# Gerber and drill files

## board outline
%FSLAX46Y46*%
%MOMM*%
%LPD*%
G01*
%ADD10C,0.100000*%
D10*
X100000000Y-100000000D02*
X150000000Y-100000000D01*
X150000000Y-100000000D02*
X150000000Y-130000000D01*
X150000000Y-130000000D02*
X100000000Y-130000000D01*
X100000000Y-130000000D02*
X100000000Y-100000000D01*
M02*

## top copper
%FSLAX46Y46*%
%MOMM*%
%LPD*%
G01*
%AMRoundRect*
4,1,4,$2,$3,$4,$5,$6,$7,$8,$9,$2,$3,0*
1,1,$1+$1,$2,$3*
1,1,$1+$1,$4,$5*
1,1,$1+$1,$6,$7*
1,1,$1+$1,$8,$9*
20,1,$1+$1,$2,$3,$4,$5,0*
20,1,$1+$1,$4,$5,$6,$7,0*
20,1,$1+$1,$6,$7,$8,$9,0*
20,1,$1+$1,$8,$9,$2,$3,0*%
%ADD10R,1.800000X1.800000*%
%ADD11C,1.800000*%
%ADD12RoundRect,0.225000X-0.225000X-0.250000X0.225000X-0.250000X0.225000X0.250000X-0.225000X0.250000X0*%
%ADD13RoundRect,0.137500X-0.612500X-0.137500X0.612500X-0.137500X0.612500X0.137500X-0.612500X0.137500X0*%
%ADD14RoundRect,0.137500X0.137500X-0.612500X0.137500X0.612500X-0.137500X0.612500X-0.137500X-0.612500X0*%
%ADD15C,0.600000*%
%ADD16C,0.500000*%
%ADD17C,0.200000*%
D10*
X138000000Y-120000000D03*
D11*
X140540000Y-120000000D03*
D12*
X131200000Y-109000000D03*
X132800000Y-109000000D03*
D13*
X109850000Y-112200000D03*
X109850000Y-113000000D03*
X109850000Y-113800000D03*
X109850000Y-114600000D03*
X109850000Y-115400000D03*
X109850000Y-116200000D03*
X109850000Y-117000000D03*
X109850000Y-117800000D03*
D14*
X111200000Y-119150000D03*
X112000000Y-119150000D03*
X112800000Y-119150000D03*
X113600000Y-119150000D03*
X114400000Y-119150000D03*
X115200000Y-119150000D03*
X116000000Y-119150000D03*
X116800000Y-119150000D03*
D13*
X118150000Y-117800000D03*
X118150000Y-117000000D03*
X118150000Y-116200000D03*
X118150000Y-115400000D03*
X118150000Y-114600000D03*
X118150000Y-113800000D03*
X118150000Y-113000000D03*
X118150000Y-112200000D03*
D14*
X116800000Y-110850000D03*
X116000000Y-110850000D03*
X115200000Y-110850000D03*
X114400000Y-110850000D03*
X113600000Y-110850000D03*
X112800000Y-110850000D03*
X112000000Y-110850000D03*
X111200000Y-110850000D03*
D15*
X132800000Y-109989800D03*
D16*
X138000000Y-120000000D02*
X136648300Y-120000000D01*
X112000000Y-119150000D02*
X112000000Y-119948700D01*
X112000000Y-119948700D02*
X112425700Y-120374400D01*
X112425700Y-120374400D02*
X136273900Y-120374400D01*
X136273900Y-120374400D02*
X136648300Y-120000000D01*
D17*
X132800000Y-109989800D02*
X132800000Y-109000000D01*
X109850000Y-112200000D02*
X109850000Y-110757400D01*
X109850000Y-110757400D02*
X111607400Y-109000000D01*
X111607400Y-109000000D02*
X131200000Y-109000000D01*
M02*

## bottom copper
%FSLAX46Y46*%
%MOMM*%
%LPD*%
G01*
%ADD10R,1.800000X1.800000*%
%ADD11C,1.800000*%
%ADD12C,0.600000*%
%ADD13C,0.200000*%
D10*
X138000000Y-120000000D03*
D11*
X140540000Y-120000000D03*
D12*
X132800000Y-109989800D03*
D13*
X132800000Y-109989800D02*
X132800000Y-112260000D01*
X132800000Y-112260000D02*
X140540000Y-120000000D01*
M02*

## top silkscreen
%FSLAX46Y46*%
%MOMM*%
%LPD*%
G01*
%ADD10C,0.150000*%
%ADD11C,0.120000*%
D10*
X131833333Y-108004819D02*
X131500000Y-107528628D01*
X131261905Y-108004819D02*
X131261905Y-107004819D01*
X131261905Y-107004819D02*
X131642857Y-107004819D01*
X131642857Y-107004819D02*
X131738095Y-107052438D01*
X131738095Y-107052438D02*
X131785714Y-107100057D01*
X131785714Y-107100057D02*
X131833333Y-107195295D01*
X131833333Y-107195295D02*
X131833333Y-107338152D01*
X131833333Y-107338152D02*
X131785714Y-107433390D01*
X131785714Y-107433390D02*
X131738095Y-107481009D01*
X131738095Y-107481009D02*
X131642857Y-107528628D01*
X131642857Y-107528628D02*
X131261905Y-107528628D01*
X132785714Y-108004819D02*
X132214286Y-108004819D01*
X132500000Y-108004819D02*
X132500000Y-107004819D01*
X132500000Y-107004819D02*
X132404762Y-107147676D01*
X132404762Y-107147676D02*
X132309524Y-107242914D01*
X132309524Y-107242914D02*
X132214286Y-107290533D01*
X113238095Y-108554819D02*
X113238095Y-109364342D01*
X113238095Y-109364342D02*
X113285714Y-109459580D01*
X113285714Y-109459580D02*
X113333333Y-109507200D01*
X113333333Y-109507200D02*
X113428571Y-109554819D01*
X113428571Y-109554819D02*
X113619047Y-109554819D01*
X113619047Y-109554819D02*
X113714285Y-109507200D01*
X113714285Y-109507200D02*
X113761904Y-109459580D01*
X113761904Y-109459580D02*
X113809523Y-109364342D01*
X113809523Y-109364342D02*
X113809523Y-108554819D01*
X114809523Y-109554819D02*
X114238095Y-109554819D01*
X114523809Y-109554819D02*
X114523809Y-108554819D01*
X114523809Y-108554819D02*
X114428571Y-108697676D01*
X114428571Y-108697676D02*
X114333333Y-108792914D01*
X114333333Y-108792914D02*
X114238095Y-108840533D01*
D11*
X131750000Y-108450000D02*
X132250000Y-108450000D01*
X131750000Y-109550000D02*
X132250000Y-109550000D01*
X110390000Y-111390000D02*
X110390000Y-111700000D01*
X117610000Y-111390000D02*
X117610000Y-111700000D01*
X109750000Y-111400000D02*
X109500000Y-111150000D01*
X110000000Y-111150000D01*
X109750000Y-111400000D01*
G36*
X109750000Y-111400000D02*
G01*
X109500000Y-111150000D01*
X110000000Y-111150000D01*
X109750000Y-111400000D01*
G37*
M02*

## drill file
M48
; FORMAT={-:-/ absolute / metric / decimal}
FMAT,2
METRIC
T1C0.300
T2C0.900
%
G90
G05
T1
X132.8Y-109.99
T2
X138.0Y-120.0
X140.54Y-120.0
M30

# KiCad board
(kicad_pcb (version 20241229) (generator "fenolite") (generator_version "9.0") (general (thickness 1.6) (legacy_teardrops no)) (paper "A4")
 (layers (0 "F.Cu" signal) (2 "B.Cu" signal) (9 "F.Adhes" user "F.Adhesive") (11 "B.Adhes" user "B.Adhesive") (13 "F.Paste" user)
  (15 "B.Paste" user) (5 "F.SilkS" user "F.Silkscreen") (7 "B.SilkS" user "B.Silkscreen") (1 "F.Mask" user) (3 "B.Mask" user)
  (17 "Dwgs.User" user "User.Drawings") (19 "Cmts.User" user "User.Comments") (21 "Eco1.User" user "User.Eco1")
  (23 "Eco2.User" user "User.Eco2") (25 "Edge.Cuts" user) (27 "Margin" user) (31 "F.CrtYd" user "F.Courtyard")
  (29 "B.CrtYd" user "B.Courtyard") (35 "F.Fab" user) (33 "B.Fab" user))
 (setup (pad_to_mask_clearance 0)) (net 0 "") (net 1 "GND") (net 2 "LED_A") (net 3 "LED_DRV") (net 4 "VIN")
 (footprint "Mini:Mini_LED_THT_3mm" (layer "B.Cu") (at 138 120)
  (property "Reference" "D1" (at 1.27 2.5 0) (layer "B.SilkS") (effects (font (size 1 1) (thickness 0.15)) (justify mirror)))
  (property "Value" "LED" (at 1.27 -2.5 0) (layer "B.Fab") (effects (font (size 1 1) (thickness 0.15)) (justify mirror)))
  (pad "1" thru_hole rect (at 0 0) (size 1.8 1.8) (drill 0.9) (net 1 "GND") (layers "*.Cu" "*.Mask") (remove_unused_layers no))
  (pad "2" thru_hole circle (at 2.54 0) (size 1.8 1.8) (drill 0.9) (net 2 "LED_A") (layers "*.Cu" "*.Mask") (remove_unused_layers no)))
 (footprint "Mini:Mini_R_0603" (layer "F.Cu") (at 132 109)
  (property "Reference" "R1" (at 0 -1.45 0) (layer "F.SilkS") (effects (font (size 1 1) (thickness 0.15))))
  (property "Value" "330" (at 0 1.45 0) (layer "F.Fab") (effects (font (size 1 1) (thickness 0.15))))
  (fp_line (start -0.25 -0.55) (end 0.25 -0.55) (stroke (width 0.12) (type solid)) (layer "F.SilkS"))
  (fp_line (start -0.25 0.55) (end 0.25 0.55) (stroke (width 0.12) (type solid)) (layer "F.SilkS"))
  (pad "1" smd roundrect (at -0.8 0) (size 0.9 0.95) (layers "F.Cu" "F.Mask" "F.Paste") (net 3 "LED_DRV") (roundrect_rratio 0.25))
  (pad "2" smd roundrect (at 0.8 0) (size 0.9 0.95) (layers "F.Cu" "F.Mask" "F.Paste") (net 2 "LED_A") (roundrect_rratio 0.25)))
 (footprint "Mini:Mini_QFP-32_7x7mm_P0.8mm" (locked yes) (layer "F.Cu") (at 114 115)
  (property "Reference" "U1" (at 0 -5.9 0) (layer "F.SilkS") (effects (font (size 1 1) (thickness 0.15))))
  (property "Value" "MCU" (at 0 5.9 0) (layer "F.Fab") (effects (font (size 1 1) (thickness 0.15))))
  (fp_line (start -3.61 -3.61) (end -3.61 -3.3) (stroke (width 0.12) (type solid)) (layer "F.SilkS"))
  (fp_line (start 3.61 -3.61) (end 3.61 -3.3) (stroke (width 0.12) (type solid)) (layer "F.SilkS"))
  (fp_poly (pts (xy -4.25 -3.6) (xy -4.5 -3.85) (xy -4 -3.85)) (stroke (width 0.12) (type solid)) (fill yes) (layer "F.SilkS"))
  (pad "1" smd roundrect (at -4.15 -2.8) (size 1.5 0.55) (layers "F.Cu" "F.Mask" "F.Paste") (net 3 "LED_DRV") (roundrect_rratio 0.25))
  (pad "2" smd roundrect (at -4.15 -2) (size 1.5 0.55) (layers "F.Cu" "F.Mask" "F.Paste") (roundrect_rratio 0.25))
  (pad "3" smd roundrect (at -4.15 -1.2) (size 1.5 0.55) (layers "F.Cu" "F.Mask" "F.Paste") (roundrect_rratio 0.25))
  (pad "4" smd roundrect (at -4.15 -0.4) (size 1.5 0.55) (layers "F.Cu" "F.Mask" "F.Paste") (roundrect_rratio 0.25))
  (pad "5" smd roundrect (at -4.15 0.4) (size 1.5 0.55) (layers "F.Cu" "F.Mask" "F.Paste") (roundrect_rratio 0.25))
  (pad "6" smd roundrect (at -4.15 1.2) (size 1.5 0.55) (layers "F.Cu" "F.Mask" "F.Paste") (roundrect_rratio 0.25))
  (pad "7" smd roundrect (at -4.15 2) (size 1.5 0.55) (layers "F.Cu" "F.Mask" "F.Paste") (roundrect_rratio 0.25))
  (pad "8" smd roundrect (at -4.15 2.8) (size 1.5 0.55) (layers "F.Cu" "F.Mask" "F.Paste") (roundrect_rratio 0.25))
  (pad "9" smd roundrect (at -2.8 4.15 90) (size 1.5 0.55) (layers "F.Cu" "F.Mask" "F.Paste") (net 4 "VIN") (roundrect_rratio 0.25))
  (pad "10" smd roundrect (at -2 4.15 90) (size 1.5 0.55) (layers "F.Cu" "F.Mask" "F.Paste") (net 1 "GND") (roundrect_rratio 0.25))
  (pad "11" smd roundrect (at -1.2 4.15 90) (size 1.5 0.55) (layers "F.Cu" "F.Mask" "F.Paste") (roundrect_rratio 0.25))
  (pad "12" smd roundrect (at -0.4 4.15 90) (size 1.5 0.55) (layers "F.Cu" "F.Mask" "F.Paste") (roundrect_rratio 0.25))
  (pad "13" smd roundrect (at 0.4 4.15 90) (size 1.5 0.55) (layers "F.Cu" "F.Mask" "F.Paste") (roundrect_rratio 0.25))
  (pad "14" smd roundrect (at 1.2 4.15 90) (size 1.5 0.55) (layers "F.Cu" "F.Mask" "F.Paste") (roundrect_rratio 0.25))
  (pad "15" smd roundrect (at 2 4.15 90) (size 1.5 0.55) (layers "F.Cu" "F.Mask" "F.Paste") (roundrect_rratio 0.25))
  (pad "16" smd roundrect (at 2.8 4.15 90) (size 1.5 0.55) (layers "F.Cu" "F.Mask" "F.Paste") (roundrect_rratio 0.25))
  (pad "17" smd roundrect (at 4.15 2.8) (size 1.5 0.55) (layers "F.Cu" "F.Mask" "F.Paste") (roundrect_rratio 0.25))
  (pad "18" smd roundrect (at 4.15 2) (size 1.5 0.55) (layers "F.Cu" "F.Mask" "F.Paste") (roundrect_rratio 0.25))
  (pad "19" smd roundrect (at 4.15 1.2) (size 1.5 0.55) (layers "F.Cu" "F.Mask" "F.Paste") (roundrect_rratio 0.25))
  (pad "20" smd roundrect (at 4.15 0.4) (size 1.5 0.55) (layers "F.Cu" "F.Mask" "F.Paste") (roundrect_rratio 0.25))
  (pad "21" smd roundrect (at 4.15 -0.4) (size 1.5 0.55) (layers "F.Cu" "F.Mask" "F.Paste") (roundrect_rratio 0.25))
  (pad "22" smd roundrect (at 4.15 -1.2) (size 1.5 0.55) (layers "F.Cu" "F.Mask" "F.Paste") (roundrect_rratio 0.25))
  (pad "23" smd roundrect (at 4.15 -2) (size 1.5 0.55) (layers "F.Cu" "F.Mask" "F.Paste") (roundrect_rratio 0.25))
  (pad "24" smd roundrect (at 4.15 -2.8) (size 1.5 0.55) (layers "F.Cu" "F.Mask" "F.Paste") (roundrect_rratio 0.25))
  (pad "25" smd roundrect (at 2.8 -4.15 90) (size 1.5 0.55) (layers "F.Cu" "F.Mask" "F.Paste") (roundrect_rratio 0.25))
  (pad "26" smd roundrect (at 2 -4.15 90) (size 1.5 0.55) (layers "F.Cu" "F.Mask" "F.Paste") (roundrect_rratio 0.25))
  (pad "27" smd roundrect (at 1.2 -4.15 90) (size 1.5 0.55) (layers "F.Cu" "F.Mask" "F.Paste") (roundrect_rratio 0.25))
  (pad "28" smd roundrect (at 0.4 -4.15 90) (size 1.5 0.55) (layers "F.Cu" "F.Mask" "F.Paste") (roundrect_rratio 0.25))
  (pad "29" smd roundrect (at -0.4 -4.15 90) (size 1.5 0.55) (layers "F.Cu" "F.Mask" "F.Paste") (roundrect_rratio 0.25))
  (pad "30" smd roundrect (at -1.2 -4.15 90) (size 1.5 0.55) (layers "F.Cu" "F.Mask" "F.Paste") (roundrect_rratio 0.25))
  (pad "31" smd roundrect (at -2 -4.15 90) (size 1.5 0.55) (layers "F.Cu" "F.Mask" "F.Paste") (roundrect_rratio 0.25))
  (pad "32" smd roundrect (at -2.8 -4.15 90) (size 1.5 0.55) (layers "F.Cu" "F.Mask" "F.Paste") (roundrect_rratio 0.25)))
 (gr_line (start 100 100) (end 150 100) (stroke (width 0.1) (type solid)) (layer "Edge.Cuts"))
 (gr_line (start 150 100) (end 150 130) (stroke (width 0.1) (type solid)) (layer "Edge.Cuts"))
 (gr_line (start 150 130) (end 100 130) (stroke (width 0.1) (type solid)) (layer "Edge.Cuts"))
 (gr_line (start 100 130) (end 100 100) (stroke (width 0.1) (type solid)) (layer "Edge.Cuts"))
 (segment (start 138 120) (end 136.6483 120) (width 0.5) (layer "F.Cu") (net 1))
 (segment (start 112 119.15) (end 112 119.9487) (width 0.5) (layer "F.Cu") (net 1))
 (segment (start 112 119.9487) (end 112.4257 120.3744) (width 0.5) (layer "F.Cu") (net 1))
 (segment (start 112.4257 120.3744) (end 136.2739 120.3744) (width 0.5) (layer "F.Cu") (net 1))
 (segment (start 136.2739 120.3744) (end 136.6483 120) (width 0.5) (layer "F.Cu") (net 1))
 (segment (start 132.8 109.9898) (end 132.8 112.26) (width 0.2) (layer "B.Cu") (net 2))
 (segment (start 132.8 112.26) (end 140.54 120) (width 0.2) (layer "B.Cu") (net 2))
 (segment (start 132.8 109.9898) (end 132.8 109) (width 0.2) (layer "F.Cu") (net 2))
 (segment (start 109.85 112.2) (end 109.85 110.7574) (width 0.2) (layer "F.Cu") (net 3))
 (segment (start 109.85 110.7574) (end 111.6074 109) (width 0.2) (layer "F.Cu") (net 3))
 (segment (start 111.6074 109) (end 131.2 109) (width 0.2) (layer "F.Cu") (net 3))
 (via (at 132.8 109.9898) (size 0.6) (drill 0.3) (layers "F.Cu" "B.Cu") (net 2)))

